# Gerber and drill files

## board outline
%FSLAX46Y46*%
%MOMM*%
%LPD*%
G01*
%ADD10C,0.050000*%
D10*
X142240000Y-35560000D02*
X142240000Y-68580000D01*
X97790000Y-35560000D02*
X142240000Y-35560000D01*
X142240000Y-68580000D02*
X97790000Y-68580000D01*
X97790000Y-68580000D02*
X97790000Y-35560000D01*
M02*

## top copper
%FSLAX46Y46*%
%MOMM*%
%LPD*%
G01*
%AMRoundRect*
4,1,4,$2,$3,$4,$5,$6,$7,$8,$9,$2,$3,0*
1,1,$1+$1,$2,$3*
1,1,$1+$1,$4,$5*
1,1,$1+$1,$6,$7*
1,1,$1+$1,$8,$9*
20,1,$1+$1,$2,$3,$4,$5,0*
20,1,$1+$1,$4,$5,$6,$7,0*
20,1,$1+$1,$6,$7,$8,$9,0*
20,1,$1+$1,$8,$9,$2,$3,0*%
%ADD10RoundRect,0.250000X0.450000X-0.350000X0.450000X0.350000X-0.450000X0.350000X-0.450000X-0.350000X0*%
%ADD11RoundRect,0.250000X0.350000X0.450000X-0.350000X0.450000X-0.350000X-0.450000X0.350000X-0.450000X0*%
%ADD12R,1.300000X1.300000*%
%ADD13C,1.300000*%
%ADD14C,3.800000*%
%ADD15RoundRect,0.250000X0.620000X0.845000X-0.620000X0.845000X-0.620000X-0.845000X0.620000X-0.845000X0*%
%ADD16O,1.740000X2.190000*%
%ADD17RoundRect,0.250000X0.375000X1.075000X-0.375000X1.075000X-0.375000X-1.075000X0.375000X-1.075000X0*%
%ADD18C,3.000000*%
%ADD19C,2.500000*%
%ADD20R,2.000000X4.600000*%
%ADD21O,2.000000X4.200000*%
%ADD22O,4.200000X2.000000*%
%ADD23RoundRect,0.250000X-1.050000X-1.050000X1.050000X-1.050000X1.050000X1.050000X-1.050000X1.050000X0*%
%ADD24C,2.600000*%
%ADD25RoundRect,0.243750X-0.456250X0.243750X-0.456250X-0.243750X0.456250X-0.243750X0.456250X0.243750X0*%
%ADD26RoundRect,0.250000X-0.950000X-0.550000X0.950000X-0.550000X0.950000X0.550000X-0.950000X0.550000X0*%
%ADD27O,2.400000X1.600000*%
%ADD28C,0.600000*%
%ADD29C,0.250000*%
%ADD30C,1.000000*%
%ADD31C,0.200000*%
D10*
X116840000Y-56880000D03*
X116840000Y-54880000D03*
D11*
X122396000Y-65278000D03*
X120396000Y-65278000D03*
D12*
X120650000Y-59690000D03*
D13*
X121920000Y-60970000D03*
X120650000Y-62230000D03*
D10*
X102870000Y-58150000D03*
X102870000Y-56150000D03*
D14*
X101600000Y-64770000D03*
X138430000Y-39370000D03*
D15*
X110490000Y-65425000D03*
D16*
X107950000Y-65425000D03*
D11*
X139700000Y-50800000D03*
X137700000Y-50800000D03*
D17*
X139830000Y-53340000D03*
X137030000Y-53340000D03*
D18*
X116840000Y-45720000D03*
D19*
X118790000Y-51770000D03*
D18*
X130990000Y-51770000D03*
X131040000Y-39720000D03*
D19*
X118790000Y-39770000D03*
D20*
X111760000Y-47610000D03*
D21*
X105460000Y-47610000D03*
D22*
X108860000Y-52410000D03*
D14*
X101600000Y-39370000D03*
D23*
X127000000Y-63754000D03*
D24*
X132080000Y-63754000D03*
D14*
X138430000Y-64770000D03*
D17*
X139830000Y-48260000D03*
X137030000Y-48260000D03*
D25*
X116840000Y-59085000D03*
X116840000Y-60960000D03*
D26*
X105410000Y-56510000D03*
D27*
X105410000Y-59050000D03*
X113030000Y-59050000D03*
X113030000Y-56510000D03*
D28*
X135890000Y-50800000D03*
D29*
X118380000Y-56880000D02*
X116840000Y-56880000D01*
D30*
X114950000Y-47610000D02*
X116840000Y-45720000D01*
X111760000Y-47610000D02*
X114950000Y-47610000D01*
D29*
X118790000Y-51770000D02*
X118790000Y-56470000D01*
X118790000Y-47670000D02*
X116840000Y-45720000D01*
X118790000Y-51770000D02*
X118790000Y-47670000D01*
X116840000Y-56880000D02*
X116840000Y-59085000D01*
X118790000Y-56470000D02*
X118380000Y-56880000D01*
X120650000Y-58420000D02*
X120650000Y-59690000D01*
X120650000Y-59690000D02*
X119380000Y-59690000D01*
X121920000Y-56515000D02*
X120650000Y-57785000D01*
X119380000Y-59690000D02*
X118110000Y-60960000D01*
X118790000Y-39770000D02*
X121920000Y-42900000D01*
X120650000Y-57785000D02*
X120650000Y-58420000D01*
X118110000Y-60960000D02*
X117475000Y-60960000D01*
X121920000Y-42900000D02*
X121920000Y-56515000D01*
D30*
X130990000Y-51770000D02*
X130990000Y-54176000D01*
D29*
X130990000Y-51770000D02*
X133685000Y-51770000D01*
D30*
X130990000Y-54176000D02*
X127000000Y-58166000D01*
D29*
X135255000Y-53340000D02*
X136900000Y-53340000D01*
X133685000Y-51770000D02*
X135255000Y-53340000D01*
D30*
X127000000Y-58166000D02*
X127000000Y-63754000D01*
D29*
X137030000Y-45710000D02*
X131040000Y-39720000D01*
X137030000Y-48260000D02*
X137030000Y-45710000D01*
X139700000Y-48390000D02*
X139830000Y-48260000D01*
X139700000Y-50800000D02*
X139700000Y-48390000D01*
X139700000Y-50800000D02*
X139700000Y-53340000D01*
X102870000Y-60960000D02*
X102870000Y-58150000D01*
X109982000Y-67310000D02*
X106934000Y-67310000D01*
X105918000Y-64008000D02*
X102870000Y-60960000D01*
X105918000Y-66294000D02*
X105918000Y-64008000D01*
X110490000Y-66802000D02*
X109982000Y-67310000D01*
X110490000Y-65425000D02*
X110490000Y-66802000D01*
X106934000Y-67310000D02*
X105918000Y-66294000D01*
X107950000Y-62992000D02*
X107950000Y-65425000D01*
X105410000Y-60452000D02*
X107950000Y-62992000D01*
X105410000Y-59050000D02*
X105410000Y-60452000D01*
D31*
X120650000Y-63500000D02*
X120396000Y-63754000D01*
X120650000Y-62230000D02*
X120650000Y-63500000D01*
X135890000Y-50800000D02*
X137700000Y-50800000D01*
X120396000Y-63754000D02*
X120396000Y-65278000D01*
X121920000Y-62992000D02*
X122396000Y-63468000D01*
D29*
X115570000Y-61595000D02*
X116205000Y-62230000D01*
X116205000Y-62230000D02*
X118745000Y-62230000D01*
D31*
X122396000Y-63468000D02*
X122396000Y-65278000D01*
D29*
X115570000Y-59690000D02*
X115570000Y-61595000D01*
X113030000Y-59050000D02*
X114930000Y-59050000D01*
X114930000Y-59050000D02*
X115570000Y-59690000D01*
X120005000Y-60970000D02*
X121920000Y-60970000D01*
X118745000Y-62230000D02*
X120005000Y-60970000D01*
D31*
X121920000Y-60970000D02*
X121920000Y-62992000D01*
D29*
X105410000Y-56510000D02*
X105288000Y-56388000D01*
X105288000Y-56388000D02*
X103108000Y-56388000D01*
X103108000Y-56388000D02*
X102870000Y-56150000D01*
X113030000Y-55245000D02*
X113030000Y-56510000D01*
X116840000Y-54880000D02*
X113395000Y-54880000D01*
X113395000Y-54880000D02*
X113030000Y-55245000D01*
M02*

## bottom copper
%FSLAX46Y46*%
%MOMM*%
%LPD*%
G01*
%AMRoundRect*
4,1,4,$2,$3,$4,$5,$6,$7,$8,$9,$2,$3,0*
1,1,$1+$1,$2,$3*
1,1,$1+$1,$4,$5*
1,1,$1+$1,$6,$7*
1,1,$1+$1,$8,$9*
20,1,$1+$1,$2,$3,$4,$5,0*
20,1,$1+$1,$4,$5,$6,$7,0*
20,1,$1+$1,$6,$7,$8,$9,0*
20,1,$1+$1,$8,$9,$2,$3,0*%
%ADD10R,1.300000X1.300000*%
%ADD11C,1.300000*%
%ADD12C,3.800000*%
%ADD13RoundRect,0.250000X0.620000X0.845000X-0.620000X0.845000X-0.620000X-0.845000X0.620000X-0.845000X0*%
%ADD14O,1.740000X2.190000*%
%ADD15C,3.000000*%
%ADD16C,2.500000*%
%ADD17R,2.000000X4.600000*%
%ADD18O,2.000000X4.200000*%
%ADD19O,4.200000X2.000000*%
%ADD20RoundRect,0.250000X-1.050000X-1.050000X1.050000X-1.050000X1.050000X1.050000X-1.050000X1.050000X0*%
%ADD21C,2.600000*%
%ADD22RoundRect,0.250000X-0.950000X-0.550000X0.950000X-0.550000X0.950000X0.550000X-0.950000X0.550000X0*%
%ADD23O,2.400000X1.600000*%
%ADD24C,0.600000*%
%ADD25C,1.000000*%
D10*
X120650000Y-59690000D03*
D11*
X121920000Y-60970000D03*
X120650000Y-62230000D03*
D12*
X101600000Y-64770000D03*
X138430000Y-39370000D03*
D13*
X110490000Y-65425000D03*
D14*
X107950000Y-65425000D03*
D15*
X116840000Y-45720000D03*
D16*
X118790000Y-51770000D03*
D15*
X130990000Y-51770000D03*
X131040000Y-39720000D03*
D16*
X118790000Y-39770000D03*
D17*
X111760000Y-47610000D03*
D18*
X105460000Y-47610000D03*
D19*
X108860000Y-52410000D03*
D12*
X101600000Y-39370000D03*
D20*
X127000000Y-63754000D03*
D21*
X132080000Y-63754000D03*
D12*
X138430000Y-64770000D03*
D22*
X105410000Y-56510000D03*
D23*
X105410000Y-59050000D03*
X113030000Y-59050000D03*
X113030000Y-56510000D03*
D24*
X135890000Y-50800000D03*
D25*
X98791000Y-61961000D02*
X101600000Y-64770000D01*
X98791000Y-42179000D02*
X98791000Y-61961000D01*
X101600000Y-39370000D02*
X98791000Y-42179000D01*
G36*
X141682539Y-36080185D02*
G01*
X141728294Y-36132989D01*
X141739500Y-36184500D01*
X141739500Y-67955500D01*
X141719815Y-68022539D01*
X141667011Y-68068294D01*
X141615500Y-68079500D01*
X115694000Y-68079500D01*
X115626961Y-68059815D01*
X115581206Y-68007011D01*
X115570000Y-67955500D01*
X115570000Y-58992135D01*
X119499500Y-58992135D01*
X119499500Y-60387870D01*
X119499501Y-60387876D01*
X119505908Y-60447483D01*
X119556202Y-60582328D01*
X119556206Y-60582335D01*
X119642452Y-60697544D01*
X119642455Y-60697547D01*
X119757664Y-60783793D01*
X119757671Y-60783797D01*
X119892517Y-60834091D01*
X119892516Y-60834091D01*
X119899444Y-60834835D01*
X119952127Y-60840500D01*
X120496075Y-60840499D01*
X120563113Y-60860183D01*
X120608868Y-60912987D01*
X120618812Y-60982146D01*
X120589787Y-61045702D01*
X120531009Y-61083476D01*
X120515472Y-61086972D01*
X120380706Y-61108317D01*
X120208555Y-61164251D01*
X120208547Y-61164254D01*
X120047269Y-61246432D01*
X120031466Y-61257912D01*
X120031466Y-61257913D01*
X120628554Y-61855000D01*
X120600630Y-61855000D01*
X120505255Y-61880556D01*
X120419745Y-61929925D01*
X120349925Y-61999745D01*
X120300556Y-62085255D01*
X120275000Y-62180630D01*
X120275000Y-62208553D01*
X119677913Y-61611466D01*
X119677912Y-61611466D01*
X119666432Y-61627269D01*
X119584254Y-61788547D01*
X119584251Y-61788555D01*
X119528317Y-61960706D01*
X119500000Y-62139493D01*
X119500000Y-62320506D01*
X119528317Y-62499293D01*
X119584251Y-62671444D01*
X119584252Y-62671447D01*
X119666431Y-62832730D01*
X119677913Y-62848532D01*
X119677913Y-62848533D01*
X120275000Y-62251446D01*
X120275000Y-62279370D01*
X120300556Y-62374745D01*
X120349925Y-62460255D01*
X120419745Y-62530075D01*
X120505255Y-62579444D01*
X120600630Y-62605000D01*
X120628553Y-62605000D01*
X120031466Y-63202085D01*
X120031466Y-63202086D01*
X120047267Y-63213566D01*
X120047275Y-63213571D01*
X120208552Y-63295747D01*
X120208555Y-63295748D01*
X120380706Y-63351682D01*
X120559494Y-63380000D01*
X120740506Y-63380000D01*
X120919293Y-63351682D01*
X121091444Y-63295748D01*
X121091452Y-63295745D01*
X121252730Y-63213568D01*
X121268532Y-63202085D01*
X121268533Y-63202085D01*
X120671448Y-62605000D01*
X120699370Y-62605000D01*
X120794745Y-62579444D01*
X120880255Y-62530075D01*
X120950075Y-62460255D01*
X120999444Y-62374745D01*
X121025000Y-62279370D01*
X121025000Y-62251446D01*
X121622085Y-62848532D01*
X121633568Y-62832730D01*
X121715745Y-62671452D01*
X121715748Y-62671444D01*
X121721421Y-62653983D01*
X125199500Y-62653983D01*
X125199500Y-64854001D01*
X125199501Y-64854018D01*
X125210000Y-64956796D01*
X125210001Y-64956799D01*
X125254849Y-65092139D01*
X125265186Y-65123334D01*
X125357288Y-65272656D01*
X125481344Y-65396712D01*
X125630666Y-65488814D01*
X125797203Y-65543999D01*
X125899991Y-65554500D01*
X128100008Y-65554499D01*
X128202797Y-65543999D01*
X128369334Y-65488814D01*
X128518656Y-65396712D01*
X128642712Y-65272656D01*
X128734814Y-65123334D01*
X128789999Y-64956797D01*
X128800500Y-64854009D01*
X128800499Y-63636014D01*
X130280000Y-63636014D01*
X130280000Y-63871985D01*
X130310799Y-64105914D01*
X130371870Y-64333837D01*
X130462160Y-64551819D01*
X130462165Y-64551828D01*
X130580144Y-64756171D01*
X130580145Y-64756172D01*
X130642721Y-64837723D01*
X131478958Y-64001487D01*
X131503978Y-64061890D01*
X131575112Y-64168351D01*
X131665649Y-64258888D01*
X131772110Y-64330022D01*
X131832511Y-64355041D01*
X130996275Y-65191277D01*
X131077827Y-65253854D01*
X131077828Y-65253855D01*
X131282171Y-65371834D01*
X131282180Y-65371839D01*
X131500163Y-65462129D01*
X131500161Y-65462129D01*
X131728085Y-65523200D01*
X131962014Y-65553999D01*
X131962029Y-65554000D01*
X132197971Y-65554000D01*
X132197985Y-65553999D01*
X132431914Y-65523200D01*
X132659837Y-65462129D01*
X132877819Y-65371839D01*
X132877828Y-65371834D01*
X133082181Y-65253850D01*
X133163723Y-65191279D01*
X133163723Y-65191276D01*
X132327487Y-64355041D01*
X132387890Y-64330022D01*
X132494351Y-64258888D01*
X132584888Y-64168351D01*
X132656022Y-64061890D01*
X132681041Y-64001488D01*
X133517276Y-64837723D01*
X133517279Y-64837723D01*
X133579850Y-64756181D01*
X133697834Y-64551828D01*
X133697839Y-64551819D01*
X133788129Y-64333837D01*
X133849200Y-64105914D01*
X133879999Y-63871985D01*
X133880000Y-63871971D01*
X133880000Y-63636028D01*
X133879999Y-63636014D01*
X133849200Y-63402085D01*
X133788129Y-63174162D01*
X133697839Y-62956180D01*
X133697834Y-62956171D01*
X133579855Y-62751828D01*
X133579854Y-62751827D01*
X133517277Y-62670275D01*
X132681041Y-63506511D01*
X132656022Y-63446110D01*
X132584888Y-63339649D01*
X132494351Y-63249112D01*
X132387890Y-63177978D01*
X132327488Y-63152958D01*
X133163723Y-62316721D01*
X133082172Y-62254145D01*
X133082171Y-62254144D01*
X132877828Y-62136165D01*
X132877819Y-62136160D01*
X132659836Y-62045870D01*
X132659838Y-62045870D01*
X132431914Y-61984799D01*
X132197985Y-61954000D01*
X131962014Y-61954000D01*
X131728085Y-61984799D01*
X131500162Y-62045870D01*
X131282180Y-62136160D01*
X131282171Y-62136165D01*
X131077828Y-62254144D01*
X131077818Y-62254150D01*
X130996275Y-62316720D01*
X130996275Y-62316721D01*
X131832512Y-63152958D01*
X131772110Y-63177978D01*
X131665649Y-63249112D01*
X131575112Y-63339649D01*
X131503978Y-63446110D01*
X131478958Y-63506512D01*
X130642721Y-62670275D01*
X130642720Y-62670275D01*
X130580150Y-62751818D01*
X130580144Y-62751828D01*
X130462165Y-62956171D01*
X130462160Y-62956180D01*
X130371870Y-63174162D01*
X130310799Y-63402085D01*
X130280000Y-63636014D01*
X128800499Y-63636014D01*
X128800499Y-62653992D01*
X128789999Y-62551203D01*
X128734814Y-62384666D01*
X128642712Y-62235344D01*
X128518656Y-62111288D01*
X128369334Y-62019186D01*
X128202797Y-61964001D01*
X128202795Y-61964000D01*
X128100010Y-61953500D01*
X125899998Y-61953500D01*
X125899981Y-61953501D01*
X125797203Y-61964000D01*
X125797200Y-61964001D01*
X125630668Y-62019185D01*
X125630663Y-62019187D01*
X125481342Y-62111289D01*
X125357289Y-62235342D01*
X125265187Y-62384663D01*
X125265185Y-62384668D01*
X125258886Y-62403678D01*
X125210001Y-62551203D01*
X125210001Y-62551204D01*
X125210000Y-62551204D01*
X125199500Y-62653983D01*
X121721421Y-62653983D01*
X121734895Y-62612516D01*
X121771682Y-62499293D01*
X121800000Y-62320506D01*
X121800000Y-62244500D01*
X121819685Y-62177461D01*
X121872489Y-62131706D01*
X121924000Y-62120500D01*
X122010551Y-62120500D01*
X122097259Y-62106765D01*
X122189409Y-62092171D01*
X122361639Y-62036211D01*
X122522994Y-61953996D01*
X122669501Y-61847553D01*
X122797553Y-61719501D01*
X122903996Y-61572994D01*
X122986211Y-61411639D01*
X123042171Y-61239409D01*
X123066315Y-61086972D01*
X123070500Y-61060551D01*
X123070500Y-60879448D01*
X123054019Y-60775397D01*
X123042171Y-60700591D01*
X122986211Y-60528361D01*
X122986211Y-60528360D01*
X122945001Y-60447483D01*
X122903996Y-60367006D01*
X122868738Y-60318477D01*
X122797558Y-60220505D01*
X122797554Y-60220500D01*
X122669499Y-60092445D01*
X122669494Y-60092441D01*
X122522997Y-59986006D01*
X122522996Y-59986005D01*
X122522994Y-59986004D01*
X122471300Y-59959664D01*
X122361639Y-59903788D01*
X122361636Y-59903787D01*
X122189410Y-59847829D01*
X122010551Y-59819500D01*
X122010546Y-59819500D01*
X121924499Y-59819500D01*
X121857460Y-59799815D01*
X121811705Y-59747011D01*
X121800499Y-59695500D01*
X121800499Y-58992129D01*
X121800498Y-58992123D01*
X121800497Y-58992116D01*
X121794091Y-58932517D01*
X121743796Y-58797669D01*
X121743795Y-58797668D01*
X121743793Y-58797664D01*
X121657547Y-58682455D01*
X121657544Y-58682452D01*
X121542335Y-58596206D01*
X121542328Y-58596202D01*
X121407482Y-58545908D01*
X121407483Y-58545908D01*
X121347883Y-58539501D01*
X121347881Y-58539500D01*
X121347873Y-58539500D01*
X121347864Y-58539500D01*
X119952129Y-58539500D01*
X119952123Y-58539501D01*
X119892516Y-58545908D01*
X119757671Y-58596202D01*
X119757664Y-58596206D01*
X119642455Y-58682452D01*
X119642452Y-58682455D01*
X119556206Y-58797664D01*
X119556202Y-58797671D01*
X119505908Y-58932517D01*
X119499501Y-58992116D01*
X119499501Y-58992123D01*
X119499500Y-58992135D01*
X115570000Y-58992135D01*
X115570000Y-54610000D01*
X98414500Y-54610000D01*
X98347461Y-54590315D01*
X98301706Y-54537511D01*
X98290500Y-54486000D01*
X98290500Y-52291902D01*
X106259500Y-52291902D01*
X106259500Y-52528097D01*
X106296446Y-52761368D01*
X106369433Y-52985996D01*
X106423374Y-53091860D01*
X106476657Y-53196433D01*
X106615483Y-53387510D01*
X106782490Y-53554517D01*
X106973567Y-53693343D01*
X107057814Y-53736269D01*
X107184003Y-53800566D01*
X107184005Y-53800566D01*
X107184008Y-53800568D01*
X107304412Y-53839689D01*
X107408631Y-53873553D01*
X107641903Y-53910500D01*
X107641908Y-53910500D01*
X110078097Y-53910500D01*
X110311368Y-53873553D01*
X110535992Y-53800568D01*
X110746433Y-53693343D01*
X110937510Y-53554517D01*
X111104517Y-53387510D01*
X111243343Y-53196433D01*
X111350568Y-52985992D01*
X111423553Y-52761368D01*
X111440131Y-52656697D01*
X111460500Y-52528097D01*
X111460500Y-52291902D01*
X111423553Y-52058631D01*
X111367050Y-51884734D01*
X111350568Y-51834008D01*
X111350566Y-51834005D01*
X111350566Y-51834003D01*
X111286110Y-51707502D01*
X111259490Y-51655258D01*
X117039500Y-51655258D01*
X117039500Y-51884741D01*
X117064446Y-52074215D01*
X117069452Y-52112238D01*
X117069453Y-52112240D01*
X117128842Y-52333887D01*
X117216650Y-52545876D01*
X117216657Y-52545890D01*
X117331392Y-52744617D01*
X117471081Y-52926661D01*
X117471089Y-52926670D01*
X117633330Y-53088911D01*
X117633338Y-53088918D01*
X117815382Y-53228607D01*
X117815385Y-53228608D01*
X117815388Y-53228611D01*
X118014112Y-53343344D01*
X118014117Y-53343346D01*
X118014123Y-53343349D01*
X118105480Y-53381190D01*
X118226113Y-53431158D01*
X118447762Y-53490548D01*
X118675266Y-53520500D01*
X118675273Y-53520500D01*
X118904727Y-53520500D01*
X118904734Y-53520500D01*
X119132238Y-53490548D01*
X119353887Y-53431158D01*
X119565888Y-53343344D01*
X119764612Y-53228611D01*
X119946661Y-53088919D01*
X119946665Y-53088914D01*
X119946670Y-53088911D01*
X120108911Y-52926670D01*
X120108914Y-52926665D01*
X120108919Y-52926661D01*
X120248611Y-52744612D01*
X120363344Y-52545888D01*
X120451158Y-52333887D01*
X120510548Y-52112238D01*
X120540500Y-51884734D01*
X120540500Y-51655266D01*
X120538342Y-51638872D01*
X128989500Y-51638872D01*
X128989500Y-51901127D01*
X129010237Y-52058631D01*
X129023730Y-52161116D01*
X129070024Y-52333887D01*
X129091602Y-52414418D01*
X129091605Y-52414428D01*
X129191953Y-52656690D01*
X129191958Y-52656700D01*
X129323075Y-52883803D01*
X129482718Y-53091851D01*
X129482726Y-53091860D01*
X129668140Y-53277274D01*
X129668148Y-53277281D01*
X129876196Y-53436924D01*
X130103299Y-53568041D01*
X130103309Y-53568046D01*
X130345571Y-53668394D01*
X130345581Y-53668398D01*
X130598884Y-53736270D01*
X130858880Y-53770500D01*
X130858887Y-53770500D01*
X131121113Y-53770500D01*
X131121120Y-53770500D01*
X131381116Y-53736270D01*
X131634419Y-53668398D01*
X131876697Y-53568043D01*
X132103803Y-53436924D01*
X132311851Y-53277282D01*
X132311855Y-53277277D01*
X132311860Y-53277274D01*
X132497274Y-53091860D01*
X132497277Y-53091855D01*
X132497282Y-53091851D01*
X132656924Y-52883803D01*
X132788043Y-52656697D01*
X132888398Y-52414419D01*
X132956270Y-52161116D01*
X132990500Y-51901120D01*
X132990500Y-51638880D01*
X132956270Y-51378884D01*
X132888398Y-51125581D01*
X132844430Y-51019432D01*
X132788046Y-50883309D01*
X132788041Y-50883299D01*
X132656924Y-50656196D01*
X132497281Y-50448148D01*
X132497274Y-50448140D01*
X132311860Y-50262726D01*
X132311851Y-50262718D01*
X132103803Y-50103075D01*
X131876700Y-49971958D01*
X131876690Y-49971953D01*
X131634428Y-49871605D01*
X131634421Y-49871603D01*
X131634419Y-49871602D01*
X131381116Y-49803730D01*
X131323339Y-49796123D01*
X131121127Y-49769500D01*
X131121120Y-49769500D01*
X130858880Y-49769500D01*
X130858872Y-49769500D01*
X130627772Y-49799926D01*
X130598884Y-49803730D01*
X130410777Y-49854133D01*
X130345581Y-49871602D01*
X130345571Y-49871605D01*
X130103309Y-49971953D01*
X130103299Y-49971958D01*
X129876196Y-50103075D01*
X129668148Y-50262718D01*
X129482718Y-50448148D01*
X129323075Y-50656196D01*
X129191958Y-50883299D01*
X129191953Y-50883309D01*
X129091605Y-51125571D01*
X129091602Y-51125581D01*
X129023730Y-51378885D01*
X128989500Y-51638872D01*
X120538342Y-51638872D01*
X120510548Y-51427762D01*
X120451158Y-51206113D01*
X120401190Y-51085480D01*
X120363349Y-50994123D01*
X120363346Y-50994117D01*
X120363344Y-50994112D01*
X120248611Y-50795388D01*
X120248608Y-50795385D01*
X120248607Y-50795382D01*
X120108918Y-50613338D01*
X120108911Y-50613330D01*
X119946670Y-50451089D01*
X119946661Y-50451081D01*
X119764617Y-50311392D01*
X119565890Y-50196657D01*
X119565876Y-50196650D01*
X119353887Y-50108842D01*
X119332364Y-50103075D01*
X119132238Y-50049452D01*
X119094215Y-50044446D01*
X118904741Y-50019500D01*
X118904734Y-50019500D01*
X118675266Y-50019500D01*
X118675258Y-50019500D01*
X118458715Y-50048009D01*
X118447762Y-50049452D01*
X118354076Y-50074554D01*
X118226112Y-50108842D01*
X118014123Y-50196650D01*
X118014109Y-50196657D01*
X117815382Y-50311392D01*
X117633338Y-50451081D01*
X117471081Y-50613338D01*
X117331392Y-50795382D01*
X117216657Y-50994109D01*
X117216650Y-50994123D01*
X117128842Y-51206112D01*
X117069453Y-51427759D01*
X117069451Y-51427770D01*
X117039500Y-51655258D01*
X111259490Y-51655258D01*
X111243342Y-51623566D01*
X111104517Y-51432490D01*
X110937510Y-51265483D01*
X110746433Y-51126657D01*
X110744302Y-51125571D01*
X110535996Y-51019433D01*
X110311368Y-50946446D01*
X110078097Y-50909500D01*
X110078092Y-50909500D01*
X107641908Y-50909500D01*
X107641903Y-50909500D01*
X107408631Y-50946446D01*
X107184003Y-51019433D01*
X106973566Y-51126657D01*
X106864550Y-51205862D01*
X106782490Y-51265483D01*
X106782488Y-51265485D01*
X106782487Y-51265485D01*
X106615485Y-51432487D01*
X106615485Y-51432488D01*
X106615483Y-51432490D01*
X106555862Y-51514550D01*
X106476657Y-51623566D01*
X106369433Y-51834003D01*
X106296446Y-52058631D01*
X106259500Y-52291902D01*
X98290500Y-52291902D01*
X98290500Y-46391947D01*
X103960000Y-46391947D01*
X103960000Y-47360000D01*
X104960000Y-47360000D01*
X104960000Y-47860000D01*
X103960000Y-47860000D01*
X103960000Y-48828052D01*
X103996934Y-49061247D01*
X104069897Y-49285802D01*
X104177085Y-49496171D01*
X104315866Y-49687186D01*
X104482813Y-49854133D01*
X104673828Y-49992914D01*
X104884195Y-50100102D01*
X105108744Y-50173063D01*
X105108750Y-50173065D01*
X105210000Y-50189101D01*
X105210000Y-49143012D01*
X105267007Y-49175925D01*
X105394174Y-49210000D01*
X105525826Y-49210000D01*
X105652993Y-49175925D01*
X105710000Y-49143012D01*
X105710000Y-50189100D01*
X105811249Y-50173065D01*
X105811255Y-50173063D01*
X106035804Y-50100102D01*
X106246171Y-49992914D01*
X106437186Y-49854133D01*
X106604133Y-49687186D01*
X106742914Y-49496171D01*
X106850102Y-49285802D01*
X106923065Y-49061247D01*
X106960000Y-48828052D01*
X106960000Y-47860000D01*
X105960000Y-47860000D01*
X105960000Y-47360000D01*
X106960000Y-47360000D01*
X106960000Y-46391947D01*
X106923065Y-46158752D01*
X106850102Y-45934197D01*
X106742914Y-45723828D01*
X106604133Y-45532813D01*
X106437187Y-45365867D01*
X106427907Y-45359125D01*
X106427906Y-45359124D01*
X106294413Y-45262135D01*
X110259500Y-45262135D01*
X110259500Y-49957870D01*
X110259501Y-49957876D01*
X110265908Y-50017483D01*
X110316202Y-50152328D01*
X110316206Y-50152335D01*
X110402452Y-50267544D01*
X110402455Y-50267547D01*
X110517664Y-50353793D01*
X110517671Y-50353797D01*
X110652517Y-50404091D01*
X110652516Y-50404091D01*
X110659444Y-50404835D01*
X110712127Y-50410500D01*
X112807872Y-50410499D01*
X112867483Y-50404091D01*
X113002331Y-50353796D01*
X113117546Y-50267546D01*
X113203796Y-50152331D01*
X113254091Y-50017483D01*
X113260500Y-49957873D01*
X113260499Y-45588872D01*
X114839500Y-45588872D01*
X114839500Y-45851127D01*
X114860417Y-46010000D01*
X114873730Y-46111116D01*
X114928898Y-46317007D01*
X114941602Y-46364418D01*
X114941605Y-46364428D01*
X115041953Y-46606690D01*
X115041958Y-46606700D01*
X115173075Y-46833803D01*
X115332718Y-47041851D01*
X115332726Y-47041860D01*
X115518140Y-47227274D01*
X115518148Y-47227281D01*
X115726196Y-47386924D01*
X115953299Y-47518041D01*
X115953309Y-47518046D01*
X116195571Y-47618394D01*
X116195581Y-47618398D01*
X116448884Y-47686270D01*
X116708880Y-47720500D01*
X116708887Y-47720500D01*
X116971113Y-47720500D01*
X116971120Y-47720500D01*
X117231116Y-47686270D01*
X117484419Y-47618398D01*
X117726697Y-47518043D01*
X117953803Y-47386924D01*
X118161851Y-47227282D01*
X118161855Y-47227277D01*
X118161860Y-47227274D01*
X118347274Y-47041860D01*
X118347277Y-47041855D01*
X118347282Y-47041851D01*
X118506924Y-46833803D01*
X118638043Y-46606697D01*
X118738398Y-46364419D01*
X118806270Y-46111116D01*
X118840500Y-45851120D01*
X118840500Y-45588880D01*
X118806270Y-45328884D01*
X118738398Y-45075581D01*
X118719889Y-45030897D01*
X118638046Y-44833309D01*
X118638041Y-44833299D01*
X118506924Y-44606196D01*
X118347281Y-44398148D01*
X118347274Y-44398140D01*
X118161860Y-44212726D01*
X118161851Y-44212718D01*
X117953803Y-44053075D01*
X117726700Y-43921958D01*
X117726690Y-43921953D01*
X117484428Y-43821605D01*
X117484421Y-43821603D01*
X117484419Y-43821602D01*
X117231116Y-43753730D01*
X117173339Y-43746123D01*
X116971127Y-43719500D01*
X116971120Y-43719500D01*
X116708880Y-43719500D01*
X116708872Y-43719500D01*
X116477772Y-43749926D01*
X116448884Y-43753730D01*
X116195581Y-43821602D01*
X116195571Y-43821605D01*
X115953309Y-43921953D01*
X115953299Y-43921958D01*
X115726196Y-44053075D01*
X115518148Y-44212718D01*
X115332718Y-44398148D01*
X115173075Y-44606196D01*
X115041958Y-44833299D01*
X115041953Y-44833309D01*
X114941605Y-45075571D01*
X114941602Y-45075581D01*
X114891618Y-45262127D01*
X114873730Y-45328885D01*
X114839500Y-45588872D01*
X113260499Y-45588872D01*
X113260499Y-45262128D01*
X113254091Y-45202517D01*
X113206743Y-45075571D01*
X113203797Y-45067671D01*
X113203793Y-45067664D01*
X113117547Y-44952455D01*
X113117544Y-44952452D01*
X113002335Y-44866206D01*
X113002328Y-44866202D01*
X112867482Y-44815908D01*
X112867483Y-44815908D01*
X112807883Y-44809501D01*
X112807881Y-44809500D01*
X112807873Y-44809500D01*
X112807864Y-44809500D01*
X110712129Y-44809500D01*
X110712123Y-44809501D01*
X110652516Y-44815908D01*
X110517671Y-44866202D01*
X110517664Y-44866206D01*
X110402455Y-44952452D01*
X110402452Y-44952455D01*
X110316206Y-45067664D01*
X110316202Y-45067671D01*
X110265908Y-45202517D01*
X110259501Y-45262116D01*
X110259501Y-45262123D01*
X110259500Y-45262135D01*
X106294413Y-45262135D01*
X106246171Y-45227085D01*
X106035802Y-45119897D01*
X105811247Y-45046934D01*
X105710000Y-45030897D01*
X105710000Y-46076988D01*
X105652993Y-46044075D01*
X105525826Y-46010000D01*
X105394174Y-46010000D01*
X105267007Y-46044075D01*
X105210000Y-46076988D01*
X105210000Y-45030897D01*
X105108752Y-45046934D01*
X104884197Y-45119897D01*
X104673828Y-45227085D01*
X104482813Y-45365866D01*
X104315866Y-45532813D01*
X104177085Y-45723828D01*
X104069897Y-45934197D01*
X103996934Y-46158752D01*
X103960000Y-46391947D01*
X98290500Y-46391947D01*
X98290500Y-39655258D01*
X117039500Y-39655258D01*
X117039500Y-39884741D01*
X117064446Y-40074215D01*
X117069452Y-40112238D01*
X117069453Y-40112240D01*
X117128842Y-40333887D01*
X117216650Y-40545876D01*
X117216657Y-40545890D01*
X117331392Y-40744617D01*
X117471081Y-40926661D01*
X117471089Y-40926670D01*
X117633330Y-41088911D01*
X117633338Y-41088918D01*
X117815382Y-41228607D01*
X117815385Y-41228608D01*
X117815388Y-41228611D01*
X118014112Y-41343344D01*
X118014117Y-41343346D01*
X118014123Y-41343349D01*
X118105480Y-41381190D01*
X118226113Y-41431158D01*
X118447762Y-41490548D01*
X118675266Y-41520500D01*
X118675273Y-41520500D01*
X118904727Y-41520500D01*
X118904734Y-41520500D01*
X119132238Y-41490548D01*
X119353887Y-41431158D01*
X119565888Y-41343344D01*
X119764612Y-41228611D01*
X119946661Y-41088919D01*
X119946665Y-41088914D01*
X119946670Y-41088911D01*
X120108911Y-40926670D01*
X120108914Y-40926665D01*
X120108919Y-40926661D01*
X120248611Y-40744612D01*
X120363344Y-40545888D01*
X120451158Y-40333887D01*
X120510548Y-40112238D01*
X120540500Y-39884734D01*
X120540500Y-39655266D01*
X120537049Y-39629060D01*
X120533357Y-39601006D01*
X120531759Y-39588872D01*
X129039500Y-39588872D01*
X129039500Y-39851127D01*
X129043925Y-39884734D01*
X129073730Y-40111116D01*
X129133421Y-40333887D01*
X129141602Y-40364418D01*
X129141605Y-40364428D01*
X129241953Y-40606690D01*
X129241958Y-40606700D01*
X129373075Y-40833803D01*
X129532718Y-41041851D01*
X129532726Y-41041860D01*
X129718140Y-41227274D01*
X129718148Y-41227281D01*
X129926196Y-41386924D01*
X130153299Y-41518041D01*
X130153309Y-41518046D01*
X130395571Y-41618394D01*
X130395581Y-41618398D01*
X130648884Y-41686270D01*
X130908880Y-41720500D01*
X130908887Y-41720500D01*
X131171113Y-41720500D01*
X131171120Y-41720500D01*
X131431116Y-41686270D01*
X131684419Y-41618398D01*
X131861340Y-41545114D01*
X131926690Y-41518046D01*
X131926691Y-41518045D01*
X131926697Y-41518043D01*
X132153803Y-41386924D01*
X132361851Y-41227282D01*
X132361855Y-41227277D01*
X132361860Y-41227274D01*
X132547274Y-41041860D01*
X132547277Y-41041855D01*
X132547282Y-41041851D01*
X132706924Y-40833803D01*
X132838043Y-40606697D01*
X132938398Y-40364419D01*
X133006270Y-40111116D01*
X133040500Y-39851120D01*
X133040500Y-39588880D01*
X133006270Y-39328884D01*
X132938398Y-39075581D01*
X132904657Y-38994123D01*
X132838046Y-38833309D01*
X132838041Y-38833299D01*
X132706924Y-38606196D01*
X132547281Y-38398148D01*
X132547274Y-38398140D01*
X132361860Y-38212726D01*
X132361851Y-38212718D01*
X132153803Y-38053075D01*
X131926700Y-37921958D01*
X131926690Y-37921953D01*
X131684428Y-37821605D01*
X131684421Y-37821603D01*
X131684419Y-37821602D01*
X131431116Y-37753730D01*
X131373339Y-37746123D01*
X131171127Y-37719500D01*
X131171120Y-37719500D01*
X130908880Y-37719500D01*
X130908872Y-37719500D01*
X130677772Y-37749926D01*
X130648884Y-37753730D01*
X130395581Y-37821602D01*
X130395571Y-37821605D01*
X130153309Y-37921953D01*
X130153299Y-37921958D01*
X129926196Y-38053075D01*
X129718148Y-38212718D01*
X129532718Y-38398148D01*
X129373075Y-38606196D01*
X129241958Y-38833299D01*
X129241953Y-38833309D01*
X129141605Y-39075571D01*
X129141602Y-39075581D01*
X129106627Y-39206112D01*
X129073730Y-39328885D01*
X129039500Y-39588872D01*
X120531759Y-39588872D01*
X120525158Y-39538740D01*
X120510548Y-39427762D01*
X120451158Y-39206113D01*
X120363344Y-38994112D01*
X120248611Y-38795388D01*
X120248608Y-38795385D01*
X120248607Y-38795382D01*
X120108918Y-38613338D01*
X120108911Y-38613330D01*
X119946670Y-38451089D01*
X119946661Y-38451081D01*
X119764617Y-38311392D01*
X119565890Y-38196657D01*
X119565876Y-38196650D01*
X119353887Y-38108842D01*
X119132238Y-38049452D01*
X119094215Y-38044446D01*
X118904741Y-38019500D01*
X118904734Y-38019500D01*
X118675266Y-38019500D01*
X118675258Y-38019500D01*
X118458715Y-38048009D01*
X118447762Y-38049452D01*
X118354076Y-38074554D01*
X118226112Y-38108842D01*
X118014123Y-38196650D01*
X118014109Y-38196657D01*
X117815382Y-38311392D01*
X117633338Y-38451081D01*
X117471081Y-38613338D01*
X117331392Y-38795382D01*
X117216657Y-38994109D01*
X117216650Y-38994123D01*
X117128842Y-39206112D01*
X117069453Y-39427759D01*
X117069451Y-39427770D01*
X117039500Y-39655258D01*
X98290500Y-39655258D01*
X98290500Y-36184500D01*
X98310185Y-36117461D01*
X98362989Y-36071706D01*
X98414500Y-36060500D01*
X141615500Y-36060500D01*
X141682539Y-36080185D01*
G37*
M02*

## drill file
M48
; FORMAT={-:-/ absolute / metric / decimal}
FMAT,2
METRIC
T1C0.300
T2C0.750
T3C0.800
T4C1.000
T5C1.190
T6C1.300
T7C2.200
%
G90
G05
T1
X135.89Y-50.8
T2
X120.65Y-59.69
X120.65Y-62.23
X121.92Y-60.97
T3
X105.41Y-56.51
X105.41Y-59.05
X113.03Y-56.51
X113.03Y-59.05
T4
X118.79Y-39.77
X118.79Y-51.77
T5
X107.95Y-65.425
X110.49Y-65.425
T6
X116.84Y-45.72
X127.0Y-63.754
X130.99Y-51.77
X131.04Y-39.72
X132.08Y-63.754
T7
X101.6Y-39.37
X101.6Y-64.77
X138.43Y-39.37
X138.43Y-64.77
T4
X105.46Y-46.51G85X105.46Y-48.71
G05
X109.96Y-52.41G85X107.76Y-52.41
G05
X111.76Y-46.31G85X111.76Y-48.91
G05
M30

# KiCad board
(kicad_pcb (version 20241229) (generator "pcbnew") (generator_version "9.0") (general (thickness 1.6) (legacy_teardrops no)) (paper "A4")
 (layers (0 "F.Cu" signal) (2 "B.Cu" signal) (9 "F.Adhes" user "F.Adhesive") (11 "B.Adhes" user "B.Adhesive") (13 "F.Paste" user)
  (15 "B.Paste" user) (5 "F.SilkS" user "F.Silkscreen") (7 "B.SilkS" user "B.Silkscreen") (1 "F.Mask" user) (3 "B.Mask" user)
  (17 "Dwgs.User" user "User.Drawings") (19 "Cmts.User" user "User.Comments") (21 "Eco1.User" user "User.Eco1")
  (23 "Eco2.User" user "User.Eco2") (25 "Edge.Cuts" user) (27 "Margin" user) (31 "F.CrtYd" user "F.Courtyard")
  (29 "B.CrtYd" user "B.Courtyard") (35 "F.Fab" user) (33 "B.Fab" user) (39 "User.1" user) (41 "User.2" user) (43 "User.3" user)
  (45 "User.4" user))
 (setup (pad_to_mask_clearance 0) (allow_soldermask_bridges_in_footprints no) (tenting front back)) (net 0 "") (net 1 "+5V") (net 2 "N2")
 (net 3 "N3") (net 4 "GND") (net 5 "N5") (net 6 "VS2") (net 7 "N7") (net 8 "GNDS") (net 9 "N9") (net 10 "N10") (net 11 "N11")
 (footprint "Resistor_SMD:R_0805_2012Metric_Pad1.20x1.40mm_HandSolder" (layer "F.Cu") (at 116.84 55.88 90)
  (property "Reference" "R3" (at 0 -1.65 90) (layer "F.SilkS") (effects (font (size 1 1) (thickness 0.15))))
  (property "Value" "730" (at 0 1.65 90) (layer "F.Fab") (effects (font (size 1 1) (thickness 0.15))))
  (pad "1" smd roundrect (at -1 0 90) (size 1.2 1.4) (layers "F.Cu" "F.Mask" "F.Paste") (roundrect_rratio 0.208333) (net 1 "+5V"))
  (pad "2" smd roundrect (at 1 0 90) (size 1.2 1.4) (layers "F.Cu" "F.Mask" "F.Paste") (roundrect_rratio 0.208333) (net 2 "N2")))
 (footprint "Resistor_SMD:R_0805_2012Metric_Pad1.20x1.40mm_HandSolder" (layer "F.Cu") (at 121.396 65.278 180)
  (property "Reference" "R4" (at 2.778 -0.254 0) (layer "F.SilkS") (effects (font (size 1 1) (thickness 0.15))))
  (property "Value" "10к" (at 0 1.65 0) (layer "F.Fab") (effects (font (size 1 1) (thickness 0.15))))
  (pad "1" smd roundrect (at -1 0 180) (size 1.2 1.4) (layers "F.Cu" "F.Mask" "F.Paste") (roundrect_rratio 0.208333) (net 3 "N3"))
  (pad "2" smd roundrect (at 1 0 180) (size 1.2 1.4) (layers "F.Cu" "F.Mask" "F.Paste") (roundrect_rratio 0.208333) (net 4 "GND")))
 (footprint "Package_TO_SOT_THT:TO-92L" (layer "F.Cu") (at 120.65 59.69 -90)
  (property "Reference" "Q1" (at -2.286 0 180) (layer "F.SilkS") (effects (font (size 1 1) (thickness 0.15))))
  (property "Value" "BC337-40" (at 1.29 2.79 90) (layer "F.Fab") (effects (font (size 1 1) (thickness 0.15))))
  (pad "1" thru_hole rect (at 0 0 270) (size 1.3 1.3) (drill 0.75) (layers "*.Cu" "*.Mask") (remove_unused_layers no) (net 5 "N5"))
  (pad "2" thru_hole circle (at 1.28 -1.27 270) (size 1.3 1.3) (drill 0.75) (layers "*.Cu" "*.Mask") (remove_unused_layers no) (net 3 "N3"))
  (pad "3" thru_hole circle (at 2.54 0 270) (size 1.3 1.3) (drill 0.75) (layers "*.Cu" "*.Mask") (remove_unused_layers no) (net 4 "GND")))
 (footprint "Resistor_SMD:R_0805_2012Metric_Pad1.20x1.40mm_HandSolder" (layer "F.Cu") (at 102.87 57.15 90)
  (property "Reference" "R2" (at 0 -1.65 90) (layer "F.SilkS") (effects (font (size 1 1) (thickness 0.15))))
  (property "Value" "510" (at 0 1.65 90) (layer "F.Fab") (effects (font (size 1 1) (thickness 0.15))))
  (pad "1" smd roundrect (at -1 0 90) (size 1.2 1.4) (layers "F.Cu" "F.Mask" "F.Paste") (roundrect_rratio 0.208333) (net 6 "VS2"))
  (pad "2" smd roundrect (at 1 0 90) (size 1.2 1.4) (layers "F.Cu" "F.Mask" "F.Paste") (roundrect_rratio 0.208333) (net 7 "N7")))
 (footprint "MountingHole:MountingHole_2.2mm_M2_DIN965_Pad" (layer "F.Cu") (at 101.6 64.77)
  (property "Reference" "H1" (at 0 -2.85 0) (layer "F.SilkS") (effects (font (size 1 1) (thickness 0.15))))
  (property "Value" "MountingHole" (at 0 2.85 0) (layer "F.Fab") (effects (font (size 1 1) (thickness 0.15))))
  (pad "1" thru_hole circle (at 0 0) (size 3.8 3.8) (drill 2.2) (layers "*.Cu" "*.Mask") (remove_unused_layers no) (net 4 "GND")
   (zone_connect 2)))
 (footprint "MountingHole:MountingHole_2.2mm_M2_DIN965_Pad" (layer "F.Cu") (at 138.43 39.37)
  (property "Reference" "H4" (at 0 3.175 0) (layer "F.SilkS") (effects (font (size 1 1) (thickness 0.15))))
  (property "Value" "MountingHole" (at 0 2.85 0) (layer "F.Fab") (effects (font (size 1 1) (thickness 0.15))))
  (pad "1" thru_hole circle (at 0 0) (size 3.8 3.8) (drill 2.2) (layers "*.Cu" "*.Mask") (remove_unused_layers no) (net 4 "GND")
   (zone_connect 2)))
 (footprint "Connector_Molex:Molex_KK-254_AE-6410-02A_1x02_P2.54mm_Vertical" (layer "F.Cu") (at 110.49 65.425 180)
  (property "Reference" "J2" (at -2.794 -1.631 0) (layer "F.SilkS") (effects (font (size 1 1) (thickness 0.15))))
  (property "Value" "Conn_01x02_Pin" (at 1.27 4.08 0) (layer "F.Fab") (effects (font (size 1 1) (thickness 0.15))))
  (pad "1" thru_hole roundrect (at 0 0 180) (size 1.74 2.19) (drill 1.19) (layers "*.Cu" "*.Mask") (remove_unused_layers no)
   (roundrect_rratio 0.143678) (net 6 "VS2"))
  (pad "2" thru_hole oval (at 2.54 0 180) (size 1.74 2.19) (drill 1.19) (layers "*.Cu" "*.Mask") (remove_unused_layers no) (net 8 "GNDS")))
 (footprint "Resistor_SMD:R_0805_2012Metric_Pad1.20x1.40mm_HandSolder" (layer "F.Cu") (at 138.7 50.8 180)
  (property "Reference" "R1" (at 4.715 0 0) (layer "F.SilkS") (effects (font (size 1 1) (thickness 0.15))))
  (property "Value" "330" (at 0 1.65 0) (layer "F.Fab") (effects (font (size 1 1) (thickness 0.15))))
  (pad "1" smd roundrect (at -1 0 180) (size 1.2 1.4) (layers "F.Cu" "F.Mask" "F.Paste") (roundrect_rratio 0.208333) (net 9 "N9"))
  (pad "2" smd roundrect (at 1 0 180) (size 1.2 1.4) (layers "F.Cu" "F.Mask" "F.Paste") (roundrect_rratio 0.208333) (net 4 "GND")))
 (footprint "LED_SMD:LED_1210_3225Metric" (layer "F.Cu") (at 138.43 53.34 180)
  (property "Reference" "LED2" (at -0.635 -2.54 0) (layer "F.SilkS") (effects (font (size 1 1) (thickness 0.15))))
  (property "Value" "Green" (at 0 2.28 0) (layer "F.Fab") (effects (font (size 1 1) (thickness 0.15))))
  (pad "1" smd roundrect (at -1.4 0 180) (size 1.25 2.65) (layers "F.Cu" "F.Mask" "F.Paste") (roundrect_rratio 0.2) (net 9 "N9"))
  (pad "2" smd roundrect (at 1.4 0 180) (size 1.25 2.65) (layers "F.Cu" "F.Mask" "F.Paste") (roundrect_rratio 0.2) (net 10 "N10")))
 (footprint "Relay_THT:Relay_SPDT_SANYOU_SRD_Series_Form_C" (layer "F.Cu") (at 116.84 45.72)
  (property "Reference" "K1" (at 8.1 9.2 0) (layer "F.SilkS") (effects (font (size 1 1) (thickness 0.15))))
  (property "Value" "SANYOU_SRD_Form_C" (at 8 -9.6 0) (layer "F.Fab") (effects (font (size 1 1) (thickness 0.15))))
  (pad "1" thru_hole circle (at 0 0 90) (size 3 3) (drill 1.3) (layers "*.Cu" "*.Mask") (remove_unused_layers no) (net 1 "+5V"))
  (pad "2" thru_hole circle (at 1.95 6.05 90) (size 2.5 2.5) (drill 1) (layers "*.Cu" "*.Mask") (remove_unused_layers no) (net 1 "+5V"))
  (pad "3" thru_hole circle (at 14.15 6.05 90) (size 3 3) (drill 1.3) (layers "*.Cu" "*.Mask") (remove_unused_layers no) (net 10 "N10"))
  (pad "4" thru_hole circle (at 14.2 -6 90) (size 3 3) (drill 1.3) (layers "*.Cu" "*.Mask") (remove_unused_layers no) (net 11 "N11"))
  (pad "5" thru_hole circle (at 1.95 -5.95 90) (size 2.5 2.5) (drill 1) (layers "*.Cu" "*.Mask") (remove_unused_layers no) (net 5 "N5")))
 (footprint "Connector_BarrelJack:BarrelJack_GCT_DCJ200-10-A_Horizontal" (layer "F.Cu") (at 111.76 47.61 -90)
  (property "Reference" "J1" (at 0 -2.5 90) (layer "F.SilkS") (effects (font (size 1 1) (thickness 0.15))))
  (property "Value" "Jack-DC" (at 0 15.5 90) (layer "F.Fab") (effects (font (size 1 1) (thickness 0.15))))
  (pad "1" thru_hole rect (at 0 0 270) (size 4.6 2) (drill oval 3.6 1) (layers "*.Cu" "*.Mask") (remove_unused_layers no) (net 1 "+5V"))
  (pad "2" thru_hole oval (at 0 6.3 270) (size 4.2 2) (drill oval 3.2 1) (layers "*.Cu" "*.Mask") (remove_unused_layers no) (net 4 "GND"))
  (pad "3" thru_hole oval (at 4.8 2.9 270) (size 2 4.2) (drill oval 1 3.2) (layers "*.Cu" "*.Mask") (remove_unused_layers no)))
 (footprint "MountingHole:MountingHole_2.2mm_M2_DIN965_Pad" (layer "F.Cu") (at 101.6 39.37)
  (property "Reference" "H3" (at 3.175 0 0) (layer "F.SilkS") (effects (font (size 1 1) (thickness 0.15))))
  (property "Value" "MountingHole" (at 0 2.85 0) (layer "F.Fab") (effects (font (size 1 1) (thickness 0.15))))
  (pad "1" thru_hole circle (at 0 0) (size 3.8 3.8) (drill 2.2) (layers "*.Cu" "*.Mask") (remove_unused_layers no) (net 4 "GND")
   (zone_connect 2)))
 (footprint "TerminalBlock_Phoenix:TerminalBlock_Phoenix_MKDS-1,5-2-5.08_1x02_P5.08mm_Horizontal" (layer "F.Cu") (at 127 63.754)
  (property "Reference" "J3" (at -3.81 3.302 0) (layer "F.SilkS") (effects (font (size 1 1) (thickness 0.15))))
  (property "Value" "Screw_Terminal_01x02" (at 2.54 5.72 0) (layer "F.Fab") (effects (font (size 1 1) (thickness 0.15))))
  (pad "1" thru_hole roundrect (at 0 0) (size 2.6 2.6) (drill 1.3) (layers "*.Cu" "*.Mask") (remove_unused_layers no)
   (roundrect_rratio 0.096154) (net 10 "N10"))
  (pad "2" thru_hole circle (at 5.08 0) (size 2.6 2.6) (drill 1.3) (layers "*.Cu" "*.Mask") (remove_unused_layers no) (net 4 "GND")))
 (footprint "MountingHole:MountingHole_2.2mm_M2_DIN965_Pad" (layer "F.Cu") (at 138.43 64.77)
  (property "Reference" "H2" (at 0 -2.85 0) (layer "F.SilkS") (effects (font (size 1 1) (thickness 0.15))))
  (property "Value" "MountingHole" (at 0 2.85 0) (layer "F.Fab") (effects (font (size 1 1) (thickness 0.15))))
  (pad "1" thru_hole circle (at 0 0) (size 3.8 3.8) (drill 2.2) (layers "*.Cu" "*.Mask") (remove_unused_layers no) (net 4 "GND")
   (zone_connect 2)))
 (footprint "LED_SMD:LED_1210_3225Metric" (layer "F.Cu") (at 138.43 48.26 180)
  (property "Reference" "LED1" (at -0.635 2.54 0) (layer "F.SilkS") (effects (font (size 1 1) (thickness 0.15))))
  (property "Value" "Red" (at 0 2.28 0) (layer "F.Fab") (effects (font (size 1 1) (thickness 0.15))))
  (pad "1" smd roundrect (at -1.4 0 180) (size 1.25 2.65) (layers "F.Cu" "F.Mask" "F.Paste") (roundrect_rratio 0.2) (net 9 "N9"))
  (pad "2" smd roundrect (at 1.4 0 180) (size 1.25 2.65) (layers "F.Cu" "F.Mask" "F.Paste") (roundrect_rratio 0.2) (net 11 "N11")))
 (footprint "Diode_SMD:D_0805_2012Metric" (layer "F.Cu") (at 116.84 60.0225 -90)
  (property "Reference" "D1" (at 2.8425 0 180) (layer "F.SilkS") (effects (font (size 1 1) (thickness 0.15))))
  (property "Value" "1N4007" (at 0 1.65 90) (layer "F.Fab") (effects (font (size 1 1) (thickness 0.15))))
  (pad "1" smd roundrect (at -0.9375 0 270) (size 0.975 1.4) (layers "F.Cu" "F.Mask" "F.Paste") (roundrect_rratio 0.25) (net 1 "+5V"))
  (pad "2" smd roundrect (at 0.9375 0 270) (size 0.975 1.4) (layers "F.Cu" "F.Mask" "F.Paste") (roundrect_rratio 0.25) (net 5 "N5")))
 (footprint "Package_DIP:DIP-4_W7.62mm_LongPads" (layer "F.Cu") (at 105.41 56.51)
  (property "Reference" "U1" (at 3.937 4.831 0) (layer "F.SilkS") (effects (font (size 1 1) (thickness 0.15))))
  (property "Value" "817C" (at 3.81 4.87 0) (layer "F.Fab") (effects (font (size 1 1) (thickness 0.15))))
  (pad "1" thru_hole roundrect (at 0 0) (size 2.4 1.6) (drill 0.8) (layers "*.Cu" "*.Mask") (remove_unused_layers no)
   (roundrect_rratio 0.15625) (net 7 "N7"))
  (pad "2" thru_hole oval (at 0 2.54) (size 2.4 1.6) (drill 0.8) (layers "*.Cu" "*.Mask") (remove_unused_layers no) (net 8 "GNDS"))
  (pad "3" thru_hole oval (at 7.62 2.54) (size 2.4 1.6) (drill 0.8) (layers "*.Cu" "*.Mask") (remove_unused_layers no) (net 3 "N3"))
  (pad "4" thru_hole oval (at 7.62 0) (size 2.4 1.6) (drill 0.8) (layers "*.Cu" "*.Mask") (remove_unused_layers no) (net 2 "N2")))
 (gr_line (start 142.24 35.56) (end 142.24 68.58) (stroke (width 0.05) (type default)) (layer "Edge.Cuts"))
 (gr_line (start 97.79 35.56) (end 142.24 35.56) (stroke (width 0.05) (type default)) (layer "Edge.Cuts"))
 (gr_line (start 142.24 68.58) (end 97.79 68.58) (stroke (width 0.05) (type default)) (layer "Edge.Cuts"))
 (gr_line (start 97.79 68.58) (end 97.79 35.56) (stroke (width 0.05) (type default)) (layer "Edge.Cuts"))
 (segment (start 118.38 56.88) (end 116.84 56.88) (width 0.25) (layer "F.Cu") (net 1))
 (segment (start 114.95 47.61) (end 116.84 45.72) (width 1) (layer "F.Cu") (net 1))
 (segment (start 111.76 47.61) (end 114.95 47.61) (width 1) (layer "F.Cu") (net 1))
 (segment (start 118.79 51.77) (end 118.79 56.47) (width 0.25) (layer "F.Cu") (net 1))
 (segment (start 118.79 47.67) (end 116.84 45.72) (width 0.25) (layer "F.Cu") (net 1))
 (segment (start 118.79 51.77) (end 118.79 47.67) (width 0.25) (layer "F.Cu") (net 1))
 (segment (start 116.84 56.88) (end 116.84 59.085) (width 0.25) (layer "F.Cu") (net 1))
 (segment (start 118.79 56.47) (end 118.38 56.88) (width 0.25) (layer "F.Cu") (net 1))
 (segment (start 120.65 58.42) (end 120.65 59.69) (width 0.25) (layer "F.Cu") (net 5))
 (segment (start 120.65 59.69) (end 119.38 59.69) (width 0.25) (layer "F.Cu") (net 5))
 (segment (start 121.92 56.515) (end 120.65 57.785) (width 0.25) (layer "F.Cu") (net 5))
 (segment (start 119.38 59.69) (end 118.11 60.96) (width 0.25) (layer "F.Cu") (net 5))
 (segment (start 118.79 39.77) (end 121.92 42.9) (width 0.25) (layer "F.Cu") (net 5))
 (segment (start 120.65 57.785) (end 120.65 58.42) (width 0.25) (layer "F.Cu") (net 5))
 (segment (start 118.11 60.96) (end 117.475 60.96) (width 0.25) (layer "F.Cu") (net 5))
 (segment (start 121.92 42.9) (end 121.92 56.515) (width 0.25) (layer "F.Cu") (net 5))
 (segment (start 130.99 51.77) (end 130.99 54.176) (width 1) (layer "F.Cu") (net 10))
 (segment (start 130.99 51.77) (end 133.685 51.77) (width 0.25) (layer "F.Cu") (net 10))
 (segment (start 130.99 54.176) (end 127 58.166) (width 1) (layer "F.Cu") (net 10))
 (segment (start 135.255 53.34) (end 136.9 53.34) (width 0.25) (layer "F.Cu") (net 10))
 (segment (start 133.685 51.77) (end 135.255 53.34) (width 0.25) (layer "F.Cu") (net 10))
 (segment (start 127 58.166) (end 127 63.754) (width 1) (layer "F.Cu") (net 10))
 (segment (start 137.03 45.71) (end 131.04 39.72) (width 0.25) (layer "F.Cu") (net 11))
 (segment (start 137.03 48.26) (end 137.03 45.71) (width 0.25) (layer "F.Cu") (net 11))
 (segment (start 139.7 48.39) (end 139.83 48.26) (width 0.25) (layer "F.Cu") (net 9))
 (segment (start 139.7 50.8) (end 139.7 48.39) (width 0.25) (layer "F.Cu") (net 9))
 (segment (start 139.7 50.8) (end 139.7 53.34) (width 0.25) (layer "F.Cu") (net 9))
 (segment (start 102.87 60.96) (end 102.87 58.15) (width 0.25) (layer "F.Cu") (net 6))
 (segment (start 109.982 67.31) (end 106.934 67.31) (width 0.25) (layer "F.Cu") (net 6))
 (segment (start 105.918 64.008) (end 102.87 60.96) (width 0.25) (layer "F.Cu") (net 6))
 (segment (start 105.918 66.294) (end 105.918 64.008) (width 0.25) (layer "F.Cu") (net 6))
 (segment (start 110.49 66.802) (end 109.982 67.31) (width 0.25) (layer "F.Cu") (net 6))
 (segment (start 110.49 65.425) (end 110.49 66.802) (width 0.25) (layer "F.Cu") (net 6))
 (segment (start 106.934 67.31) (end 105.918 66.294) (width 0.25) (layer "F.Cu") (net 6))
 (segment (start 107.95 62.992) (end 107.95 65.425) (width 0.25) (layer "F.Cu") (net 8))
 (segment (start 105.41 60.452) (end 107.95 62.992) (width 0.25) (layer "F.Cu") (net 8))
 (segment (start 105.41 59.05) (end 105.41 60.452) (width 0.25) (layer "F.Cu") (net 8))
 (segment (start 120.65 63.5) (end 120.396 63.754) (width 0.2) (layer "F.Cu") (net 4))
 (segment (start 120.65 62.23) (end 120.65 63.5) (width 0.2) (layer "F.Cu") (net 4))
 (segment (start 135.89 50.8) (end 137.7 50.8) (width 0.2) (layer "F.Cu") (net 4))
 (segment (start 120.396 63.754) (end 120.396 65.278) (width 0.2) (layer "F.Cu") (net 4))
 (via (at 135.89 50.8) (size 0.6) (drill 0.3) (layers "F.Cu" "B.Cu") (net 4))
 (segment (start 98.791 61.961) (end 101.6 64.77) (width 1) (layer "B.Cu") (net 4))
 (segment (start 98.791 42.179) (end 98.791 61.961) (width 1) (layer "B.Cu") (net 4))
 (segment (start 101.6 39.37) (end 98.791 42.179) (width 1) (layer "B.Cu") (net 4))
 (segment (start 121.92 62.992) (end 122.396 63.468) (width 0.2) (layer "F.Cu") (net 3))
 (segment (start 115.57 61.595) (end 116.205 62.23) (width 0.25) (layer "F.Cu") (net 3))
 (segment (start 116.205 62.23) (end 118.745 62.23) (width 0.25) (layer "F.Cu") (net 3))
 (segment (start 122.396 63.468) (end 122.396 65.278) (width 0.2) (layer "F.Cu") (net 3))
 (segment (start 115.57 59.69) (end 115.57 61.595) (width 0.25) (layer "F.Cu") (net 3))
 (segment (start 113.03 59.05) (end 114.93 59.05) (width 0.25) (layer "F.Cu") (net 3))
 (segment (start 114.93 59.05) (end 115.57 59.69) (width 0.25) (layer "F.Cu") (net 3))
 (segment (start 120.005 60.97) (end 121.92 60.97) (width 0.25) (layer "F.Cu") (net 3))
 (segment (start 118.745 62.23) (end 120.005 60.97) (width 0.25) (layer "F.Cu") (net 3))
 (segment (start 121.92 60.97) (end 121.92 62.992) (width 0.2) (layer "F.Cu") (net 3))
 (segment (start 105.41 56.51) (end 105.288 56.388) (width 0.25) (layer "F.Cu") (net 7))
 (segment (start 105.288 56.388) (end 103.108 56.388) (width 0.25) (layer "F.Cu") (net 7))
 (segment (start 103.108 56.388) (end 102.87 56.15) (width 0.25) (layer "F.Cu") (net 7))
 (segment (start 113.03 55.245) (end 113.03 56.51) (width 0.25) (layer "F.Cu") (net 2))
 (segment (start 116.84 54.88) (end 113.395 54.88) (width 0.25) (layer "F.Cu") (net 2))
 (segment (start 113.395 54.88) (end 113.03 55.245) (width 0.25) (layer "F.Cu") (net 2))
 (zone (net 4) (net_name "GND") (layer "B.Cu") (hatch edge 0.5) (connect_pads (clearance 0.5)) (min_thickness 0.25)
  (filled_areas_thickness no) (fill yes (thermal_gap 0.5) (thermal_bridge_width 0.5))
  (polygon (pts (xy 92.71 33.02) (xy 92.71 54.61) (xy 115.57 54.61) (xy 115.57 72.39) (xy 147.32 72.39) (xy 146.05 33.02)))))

